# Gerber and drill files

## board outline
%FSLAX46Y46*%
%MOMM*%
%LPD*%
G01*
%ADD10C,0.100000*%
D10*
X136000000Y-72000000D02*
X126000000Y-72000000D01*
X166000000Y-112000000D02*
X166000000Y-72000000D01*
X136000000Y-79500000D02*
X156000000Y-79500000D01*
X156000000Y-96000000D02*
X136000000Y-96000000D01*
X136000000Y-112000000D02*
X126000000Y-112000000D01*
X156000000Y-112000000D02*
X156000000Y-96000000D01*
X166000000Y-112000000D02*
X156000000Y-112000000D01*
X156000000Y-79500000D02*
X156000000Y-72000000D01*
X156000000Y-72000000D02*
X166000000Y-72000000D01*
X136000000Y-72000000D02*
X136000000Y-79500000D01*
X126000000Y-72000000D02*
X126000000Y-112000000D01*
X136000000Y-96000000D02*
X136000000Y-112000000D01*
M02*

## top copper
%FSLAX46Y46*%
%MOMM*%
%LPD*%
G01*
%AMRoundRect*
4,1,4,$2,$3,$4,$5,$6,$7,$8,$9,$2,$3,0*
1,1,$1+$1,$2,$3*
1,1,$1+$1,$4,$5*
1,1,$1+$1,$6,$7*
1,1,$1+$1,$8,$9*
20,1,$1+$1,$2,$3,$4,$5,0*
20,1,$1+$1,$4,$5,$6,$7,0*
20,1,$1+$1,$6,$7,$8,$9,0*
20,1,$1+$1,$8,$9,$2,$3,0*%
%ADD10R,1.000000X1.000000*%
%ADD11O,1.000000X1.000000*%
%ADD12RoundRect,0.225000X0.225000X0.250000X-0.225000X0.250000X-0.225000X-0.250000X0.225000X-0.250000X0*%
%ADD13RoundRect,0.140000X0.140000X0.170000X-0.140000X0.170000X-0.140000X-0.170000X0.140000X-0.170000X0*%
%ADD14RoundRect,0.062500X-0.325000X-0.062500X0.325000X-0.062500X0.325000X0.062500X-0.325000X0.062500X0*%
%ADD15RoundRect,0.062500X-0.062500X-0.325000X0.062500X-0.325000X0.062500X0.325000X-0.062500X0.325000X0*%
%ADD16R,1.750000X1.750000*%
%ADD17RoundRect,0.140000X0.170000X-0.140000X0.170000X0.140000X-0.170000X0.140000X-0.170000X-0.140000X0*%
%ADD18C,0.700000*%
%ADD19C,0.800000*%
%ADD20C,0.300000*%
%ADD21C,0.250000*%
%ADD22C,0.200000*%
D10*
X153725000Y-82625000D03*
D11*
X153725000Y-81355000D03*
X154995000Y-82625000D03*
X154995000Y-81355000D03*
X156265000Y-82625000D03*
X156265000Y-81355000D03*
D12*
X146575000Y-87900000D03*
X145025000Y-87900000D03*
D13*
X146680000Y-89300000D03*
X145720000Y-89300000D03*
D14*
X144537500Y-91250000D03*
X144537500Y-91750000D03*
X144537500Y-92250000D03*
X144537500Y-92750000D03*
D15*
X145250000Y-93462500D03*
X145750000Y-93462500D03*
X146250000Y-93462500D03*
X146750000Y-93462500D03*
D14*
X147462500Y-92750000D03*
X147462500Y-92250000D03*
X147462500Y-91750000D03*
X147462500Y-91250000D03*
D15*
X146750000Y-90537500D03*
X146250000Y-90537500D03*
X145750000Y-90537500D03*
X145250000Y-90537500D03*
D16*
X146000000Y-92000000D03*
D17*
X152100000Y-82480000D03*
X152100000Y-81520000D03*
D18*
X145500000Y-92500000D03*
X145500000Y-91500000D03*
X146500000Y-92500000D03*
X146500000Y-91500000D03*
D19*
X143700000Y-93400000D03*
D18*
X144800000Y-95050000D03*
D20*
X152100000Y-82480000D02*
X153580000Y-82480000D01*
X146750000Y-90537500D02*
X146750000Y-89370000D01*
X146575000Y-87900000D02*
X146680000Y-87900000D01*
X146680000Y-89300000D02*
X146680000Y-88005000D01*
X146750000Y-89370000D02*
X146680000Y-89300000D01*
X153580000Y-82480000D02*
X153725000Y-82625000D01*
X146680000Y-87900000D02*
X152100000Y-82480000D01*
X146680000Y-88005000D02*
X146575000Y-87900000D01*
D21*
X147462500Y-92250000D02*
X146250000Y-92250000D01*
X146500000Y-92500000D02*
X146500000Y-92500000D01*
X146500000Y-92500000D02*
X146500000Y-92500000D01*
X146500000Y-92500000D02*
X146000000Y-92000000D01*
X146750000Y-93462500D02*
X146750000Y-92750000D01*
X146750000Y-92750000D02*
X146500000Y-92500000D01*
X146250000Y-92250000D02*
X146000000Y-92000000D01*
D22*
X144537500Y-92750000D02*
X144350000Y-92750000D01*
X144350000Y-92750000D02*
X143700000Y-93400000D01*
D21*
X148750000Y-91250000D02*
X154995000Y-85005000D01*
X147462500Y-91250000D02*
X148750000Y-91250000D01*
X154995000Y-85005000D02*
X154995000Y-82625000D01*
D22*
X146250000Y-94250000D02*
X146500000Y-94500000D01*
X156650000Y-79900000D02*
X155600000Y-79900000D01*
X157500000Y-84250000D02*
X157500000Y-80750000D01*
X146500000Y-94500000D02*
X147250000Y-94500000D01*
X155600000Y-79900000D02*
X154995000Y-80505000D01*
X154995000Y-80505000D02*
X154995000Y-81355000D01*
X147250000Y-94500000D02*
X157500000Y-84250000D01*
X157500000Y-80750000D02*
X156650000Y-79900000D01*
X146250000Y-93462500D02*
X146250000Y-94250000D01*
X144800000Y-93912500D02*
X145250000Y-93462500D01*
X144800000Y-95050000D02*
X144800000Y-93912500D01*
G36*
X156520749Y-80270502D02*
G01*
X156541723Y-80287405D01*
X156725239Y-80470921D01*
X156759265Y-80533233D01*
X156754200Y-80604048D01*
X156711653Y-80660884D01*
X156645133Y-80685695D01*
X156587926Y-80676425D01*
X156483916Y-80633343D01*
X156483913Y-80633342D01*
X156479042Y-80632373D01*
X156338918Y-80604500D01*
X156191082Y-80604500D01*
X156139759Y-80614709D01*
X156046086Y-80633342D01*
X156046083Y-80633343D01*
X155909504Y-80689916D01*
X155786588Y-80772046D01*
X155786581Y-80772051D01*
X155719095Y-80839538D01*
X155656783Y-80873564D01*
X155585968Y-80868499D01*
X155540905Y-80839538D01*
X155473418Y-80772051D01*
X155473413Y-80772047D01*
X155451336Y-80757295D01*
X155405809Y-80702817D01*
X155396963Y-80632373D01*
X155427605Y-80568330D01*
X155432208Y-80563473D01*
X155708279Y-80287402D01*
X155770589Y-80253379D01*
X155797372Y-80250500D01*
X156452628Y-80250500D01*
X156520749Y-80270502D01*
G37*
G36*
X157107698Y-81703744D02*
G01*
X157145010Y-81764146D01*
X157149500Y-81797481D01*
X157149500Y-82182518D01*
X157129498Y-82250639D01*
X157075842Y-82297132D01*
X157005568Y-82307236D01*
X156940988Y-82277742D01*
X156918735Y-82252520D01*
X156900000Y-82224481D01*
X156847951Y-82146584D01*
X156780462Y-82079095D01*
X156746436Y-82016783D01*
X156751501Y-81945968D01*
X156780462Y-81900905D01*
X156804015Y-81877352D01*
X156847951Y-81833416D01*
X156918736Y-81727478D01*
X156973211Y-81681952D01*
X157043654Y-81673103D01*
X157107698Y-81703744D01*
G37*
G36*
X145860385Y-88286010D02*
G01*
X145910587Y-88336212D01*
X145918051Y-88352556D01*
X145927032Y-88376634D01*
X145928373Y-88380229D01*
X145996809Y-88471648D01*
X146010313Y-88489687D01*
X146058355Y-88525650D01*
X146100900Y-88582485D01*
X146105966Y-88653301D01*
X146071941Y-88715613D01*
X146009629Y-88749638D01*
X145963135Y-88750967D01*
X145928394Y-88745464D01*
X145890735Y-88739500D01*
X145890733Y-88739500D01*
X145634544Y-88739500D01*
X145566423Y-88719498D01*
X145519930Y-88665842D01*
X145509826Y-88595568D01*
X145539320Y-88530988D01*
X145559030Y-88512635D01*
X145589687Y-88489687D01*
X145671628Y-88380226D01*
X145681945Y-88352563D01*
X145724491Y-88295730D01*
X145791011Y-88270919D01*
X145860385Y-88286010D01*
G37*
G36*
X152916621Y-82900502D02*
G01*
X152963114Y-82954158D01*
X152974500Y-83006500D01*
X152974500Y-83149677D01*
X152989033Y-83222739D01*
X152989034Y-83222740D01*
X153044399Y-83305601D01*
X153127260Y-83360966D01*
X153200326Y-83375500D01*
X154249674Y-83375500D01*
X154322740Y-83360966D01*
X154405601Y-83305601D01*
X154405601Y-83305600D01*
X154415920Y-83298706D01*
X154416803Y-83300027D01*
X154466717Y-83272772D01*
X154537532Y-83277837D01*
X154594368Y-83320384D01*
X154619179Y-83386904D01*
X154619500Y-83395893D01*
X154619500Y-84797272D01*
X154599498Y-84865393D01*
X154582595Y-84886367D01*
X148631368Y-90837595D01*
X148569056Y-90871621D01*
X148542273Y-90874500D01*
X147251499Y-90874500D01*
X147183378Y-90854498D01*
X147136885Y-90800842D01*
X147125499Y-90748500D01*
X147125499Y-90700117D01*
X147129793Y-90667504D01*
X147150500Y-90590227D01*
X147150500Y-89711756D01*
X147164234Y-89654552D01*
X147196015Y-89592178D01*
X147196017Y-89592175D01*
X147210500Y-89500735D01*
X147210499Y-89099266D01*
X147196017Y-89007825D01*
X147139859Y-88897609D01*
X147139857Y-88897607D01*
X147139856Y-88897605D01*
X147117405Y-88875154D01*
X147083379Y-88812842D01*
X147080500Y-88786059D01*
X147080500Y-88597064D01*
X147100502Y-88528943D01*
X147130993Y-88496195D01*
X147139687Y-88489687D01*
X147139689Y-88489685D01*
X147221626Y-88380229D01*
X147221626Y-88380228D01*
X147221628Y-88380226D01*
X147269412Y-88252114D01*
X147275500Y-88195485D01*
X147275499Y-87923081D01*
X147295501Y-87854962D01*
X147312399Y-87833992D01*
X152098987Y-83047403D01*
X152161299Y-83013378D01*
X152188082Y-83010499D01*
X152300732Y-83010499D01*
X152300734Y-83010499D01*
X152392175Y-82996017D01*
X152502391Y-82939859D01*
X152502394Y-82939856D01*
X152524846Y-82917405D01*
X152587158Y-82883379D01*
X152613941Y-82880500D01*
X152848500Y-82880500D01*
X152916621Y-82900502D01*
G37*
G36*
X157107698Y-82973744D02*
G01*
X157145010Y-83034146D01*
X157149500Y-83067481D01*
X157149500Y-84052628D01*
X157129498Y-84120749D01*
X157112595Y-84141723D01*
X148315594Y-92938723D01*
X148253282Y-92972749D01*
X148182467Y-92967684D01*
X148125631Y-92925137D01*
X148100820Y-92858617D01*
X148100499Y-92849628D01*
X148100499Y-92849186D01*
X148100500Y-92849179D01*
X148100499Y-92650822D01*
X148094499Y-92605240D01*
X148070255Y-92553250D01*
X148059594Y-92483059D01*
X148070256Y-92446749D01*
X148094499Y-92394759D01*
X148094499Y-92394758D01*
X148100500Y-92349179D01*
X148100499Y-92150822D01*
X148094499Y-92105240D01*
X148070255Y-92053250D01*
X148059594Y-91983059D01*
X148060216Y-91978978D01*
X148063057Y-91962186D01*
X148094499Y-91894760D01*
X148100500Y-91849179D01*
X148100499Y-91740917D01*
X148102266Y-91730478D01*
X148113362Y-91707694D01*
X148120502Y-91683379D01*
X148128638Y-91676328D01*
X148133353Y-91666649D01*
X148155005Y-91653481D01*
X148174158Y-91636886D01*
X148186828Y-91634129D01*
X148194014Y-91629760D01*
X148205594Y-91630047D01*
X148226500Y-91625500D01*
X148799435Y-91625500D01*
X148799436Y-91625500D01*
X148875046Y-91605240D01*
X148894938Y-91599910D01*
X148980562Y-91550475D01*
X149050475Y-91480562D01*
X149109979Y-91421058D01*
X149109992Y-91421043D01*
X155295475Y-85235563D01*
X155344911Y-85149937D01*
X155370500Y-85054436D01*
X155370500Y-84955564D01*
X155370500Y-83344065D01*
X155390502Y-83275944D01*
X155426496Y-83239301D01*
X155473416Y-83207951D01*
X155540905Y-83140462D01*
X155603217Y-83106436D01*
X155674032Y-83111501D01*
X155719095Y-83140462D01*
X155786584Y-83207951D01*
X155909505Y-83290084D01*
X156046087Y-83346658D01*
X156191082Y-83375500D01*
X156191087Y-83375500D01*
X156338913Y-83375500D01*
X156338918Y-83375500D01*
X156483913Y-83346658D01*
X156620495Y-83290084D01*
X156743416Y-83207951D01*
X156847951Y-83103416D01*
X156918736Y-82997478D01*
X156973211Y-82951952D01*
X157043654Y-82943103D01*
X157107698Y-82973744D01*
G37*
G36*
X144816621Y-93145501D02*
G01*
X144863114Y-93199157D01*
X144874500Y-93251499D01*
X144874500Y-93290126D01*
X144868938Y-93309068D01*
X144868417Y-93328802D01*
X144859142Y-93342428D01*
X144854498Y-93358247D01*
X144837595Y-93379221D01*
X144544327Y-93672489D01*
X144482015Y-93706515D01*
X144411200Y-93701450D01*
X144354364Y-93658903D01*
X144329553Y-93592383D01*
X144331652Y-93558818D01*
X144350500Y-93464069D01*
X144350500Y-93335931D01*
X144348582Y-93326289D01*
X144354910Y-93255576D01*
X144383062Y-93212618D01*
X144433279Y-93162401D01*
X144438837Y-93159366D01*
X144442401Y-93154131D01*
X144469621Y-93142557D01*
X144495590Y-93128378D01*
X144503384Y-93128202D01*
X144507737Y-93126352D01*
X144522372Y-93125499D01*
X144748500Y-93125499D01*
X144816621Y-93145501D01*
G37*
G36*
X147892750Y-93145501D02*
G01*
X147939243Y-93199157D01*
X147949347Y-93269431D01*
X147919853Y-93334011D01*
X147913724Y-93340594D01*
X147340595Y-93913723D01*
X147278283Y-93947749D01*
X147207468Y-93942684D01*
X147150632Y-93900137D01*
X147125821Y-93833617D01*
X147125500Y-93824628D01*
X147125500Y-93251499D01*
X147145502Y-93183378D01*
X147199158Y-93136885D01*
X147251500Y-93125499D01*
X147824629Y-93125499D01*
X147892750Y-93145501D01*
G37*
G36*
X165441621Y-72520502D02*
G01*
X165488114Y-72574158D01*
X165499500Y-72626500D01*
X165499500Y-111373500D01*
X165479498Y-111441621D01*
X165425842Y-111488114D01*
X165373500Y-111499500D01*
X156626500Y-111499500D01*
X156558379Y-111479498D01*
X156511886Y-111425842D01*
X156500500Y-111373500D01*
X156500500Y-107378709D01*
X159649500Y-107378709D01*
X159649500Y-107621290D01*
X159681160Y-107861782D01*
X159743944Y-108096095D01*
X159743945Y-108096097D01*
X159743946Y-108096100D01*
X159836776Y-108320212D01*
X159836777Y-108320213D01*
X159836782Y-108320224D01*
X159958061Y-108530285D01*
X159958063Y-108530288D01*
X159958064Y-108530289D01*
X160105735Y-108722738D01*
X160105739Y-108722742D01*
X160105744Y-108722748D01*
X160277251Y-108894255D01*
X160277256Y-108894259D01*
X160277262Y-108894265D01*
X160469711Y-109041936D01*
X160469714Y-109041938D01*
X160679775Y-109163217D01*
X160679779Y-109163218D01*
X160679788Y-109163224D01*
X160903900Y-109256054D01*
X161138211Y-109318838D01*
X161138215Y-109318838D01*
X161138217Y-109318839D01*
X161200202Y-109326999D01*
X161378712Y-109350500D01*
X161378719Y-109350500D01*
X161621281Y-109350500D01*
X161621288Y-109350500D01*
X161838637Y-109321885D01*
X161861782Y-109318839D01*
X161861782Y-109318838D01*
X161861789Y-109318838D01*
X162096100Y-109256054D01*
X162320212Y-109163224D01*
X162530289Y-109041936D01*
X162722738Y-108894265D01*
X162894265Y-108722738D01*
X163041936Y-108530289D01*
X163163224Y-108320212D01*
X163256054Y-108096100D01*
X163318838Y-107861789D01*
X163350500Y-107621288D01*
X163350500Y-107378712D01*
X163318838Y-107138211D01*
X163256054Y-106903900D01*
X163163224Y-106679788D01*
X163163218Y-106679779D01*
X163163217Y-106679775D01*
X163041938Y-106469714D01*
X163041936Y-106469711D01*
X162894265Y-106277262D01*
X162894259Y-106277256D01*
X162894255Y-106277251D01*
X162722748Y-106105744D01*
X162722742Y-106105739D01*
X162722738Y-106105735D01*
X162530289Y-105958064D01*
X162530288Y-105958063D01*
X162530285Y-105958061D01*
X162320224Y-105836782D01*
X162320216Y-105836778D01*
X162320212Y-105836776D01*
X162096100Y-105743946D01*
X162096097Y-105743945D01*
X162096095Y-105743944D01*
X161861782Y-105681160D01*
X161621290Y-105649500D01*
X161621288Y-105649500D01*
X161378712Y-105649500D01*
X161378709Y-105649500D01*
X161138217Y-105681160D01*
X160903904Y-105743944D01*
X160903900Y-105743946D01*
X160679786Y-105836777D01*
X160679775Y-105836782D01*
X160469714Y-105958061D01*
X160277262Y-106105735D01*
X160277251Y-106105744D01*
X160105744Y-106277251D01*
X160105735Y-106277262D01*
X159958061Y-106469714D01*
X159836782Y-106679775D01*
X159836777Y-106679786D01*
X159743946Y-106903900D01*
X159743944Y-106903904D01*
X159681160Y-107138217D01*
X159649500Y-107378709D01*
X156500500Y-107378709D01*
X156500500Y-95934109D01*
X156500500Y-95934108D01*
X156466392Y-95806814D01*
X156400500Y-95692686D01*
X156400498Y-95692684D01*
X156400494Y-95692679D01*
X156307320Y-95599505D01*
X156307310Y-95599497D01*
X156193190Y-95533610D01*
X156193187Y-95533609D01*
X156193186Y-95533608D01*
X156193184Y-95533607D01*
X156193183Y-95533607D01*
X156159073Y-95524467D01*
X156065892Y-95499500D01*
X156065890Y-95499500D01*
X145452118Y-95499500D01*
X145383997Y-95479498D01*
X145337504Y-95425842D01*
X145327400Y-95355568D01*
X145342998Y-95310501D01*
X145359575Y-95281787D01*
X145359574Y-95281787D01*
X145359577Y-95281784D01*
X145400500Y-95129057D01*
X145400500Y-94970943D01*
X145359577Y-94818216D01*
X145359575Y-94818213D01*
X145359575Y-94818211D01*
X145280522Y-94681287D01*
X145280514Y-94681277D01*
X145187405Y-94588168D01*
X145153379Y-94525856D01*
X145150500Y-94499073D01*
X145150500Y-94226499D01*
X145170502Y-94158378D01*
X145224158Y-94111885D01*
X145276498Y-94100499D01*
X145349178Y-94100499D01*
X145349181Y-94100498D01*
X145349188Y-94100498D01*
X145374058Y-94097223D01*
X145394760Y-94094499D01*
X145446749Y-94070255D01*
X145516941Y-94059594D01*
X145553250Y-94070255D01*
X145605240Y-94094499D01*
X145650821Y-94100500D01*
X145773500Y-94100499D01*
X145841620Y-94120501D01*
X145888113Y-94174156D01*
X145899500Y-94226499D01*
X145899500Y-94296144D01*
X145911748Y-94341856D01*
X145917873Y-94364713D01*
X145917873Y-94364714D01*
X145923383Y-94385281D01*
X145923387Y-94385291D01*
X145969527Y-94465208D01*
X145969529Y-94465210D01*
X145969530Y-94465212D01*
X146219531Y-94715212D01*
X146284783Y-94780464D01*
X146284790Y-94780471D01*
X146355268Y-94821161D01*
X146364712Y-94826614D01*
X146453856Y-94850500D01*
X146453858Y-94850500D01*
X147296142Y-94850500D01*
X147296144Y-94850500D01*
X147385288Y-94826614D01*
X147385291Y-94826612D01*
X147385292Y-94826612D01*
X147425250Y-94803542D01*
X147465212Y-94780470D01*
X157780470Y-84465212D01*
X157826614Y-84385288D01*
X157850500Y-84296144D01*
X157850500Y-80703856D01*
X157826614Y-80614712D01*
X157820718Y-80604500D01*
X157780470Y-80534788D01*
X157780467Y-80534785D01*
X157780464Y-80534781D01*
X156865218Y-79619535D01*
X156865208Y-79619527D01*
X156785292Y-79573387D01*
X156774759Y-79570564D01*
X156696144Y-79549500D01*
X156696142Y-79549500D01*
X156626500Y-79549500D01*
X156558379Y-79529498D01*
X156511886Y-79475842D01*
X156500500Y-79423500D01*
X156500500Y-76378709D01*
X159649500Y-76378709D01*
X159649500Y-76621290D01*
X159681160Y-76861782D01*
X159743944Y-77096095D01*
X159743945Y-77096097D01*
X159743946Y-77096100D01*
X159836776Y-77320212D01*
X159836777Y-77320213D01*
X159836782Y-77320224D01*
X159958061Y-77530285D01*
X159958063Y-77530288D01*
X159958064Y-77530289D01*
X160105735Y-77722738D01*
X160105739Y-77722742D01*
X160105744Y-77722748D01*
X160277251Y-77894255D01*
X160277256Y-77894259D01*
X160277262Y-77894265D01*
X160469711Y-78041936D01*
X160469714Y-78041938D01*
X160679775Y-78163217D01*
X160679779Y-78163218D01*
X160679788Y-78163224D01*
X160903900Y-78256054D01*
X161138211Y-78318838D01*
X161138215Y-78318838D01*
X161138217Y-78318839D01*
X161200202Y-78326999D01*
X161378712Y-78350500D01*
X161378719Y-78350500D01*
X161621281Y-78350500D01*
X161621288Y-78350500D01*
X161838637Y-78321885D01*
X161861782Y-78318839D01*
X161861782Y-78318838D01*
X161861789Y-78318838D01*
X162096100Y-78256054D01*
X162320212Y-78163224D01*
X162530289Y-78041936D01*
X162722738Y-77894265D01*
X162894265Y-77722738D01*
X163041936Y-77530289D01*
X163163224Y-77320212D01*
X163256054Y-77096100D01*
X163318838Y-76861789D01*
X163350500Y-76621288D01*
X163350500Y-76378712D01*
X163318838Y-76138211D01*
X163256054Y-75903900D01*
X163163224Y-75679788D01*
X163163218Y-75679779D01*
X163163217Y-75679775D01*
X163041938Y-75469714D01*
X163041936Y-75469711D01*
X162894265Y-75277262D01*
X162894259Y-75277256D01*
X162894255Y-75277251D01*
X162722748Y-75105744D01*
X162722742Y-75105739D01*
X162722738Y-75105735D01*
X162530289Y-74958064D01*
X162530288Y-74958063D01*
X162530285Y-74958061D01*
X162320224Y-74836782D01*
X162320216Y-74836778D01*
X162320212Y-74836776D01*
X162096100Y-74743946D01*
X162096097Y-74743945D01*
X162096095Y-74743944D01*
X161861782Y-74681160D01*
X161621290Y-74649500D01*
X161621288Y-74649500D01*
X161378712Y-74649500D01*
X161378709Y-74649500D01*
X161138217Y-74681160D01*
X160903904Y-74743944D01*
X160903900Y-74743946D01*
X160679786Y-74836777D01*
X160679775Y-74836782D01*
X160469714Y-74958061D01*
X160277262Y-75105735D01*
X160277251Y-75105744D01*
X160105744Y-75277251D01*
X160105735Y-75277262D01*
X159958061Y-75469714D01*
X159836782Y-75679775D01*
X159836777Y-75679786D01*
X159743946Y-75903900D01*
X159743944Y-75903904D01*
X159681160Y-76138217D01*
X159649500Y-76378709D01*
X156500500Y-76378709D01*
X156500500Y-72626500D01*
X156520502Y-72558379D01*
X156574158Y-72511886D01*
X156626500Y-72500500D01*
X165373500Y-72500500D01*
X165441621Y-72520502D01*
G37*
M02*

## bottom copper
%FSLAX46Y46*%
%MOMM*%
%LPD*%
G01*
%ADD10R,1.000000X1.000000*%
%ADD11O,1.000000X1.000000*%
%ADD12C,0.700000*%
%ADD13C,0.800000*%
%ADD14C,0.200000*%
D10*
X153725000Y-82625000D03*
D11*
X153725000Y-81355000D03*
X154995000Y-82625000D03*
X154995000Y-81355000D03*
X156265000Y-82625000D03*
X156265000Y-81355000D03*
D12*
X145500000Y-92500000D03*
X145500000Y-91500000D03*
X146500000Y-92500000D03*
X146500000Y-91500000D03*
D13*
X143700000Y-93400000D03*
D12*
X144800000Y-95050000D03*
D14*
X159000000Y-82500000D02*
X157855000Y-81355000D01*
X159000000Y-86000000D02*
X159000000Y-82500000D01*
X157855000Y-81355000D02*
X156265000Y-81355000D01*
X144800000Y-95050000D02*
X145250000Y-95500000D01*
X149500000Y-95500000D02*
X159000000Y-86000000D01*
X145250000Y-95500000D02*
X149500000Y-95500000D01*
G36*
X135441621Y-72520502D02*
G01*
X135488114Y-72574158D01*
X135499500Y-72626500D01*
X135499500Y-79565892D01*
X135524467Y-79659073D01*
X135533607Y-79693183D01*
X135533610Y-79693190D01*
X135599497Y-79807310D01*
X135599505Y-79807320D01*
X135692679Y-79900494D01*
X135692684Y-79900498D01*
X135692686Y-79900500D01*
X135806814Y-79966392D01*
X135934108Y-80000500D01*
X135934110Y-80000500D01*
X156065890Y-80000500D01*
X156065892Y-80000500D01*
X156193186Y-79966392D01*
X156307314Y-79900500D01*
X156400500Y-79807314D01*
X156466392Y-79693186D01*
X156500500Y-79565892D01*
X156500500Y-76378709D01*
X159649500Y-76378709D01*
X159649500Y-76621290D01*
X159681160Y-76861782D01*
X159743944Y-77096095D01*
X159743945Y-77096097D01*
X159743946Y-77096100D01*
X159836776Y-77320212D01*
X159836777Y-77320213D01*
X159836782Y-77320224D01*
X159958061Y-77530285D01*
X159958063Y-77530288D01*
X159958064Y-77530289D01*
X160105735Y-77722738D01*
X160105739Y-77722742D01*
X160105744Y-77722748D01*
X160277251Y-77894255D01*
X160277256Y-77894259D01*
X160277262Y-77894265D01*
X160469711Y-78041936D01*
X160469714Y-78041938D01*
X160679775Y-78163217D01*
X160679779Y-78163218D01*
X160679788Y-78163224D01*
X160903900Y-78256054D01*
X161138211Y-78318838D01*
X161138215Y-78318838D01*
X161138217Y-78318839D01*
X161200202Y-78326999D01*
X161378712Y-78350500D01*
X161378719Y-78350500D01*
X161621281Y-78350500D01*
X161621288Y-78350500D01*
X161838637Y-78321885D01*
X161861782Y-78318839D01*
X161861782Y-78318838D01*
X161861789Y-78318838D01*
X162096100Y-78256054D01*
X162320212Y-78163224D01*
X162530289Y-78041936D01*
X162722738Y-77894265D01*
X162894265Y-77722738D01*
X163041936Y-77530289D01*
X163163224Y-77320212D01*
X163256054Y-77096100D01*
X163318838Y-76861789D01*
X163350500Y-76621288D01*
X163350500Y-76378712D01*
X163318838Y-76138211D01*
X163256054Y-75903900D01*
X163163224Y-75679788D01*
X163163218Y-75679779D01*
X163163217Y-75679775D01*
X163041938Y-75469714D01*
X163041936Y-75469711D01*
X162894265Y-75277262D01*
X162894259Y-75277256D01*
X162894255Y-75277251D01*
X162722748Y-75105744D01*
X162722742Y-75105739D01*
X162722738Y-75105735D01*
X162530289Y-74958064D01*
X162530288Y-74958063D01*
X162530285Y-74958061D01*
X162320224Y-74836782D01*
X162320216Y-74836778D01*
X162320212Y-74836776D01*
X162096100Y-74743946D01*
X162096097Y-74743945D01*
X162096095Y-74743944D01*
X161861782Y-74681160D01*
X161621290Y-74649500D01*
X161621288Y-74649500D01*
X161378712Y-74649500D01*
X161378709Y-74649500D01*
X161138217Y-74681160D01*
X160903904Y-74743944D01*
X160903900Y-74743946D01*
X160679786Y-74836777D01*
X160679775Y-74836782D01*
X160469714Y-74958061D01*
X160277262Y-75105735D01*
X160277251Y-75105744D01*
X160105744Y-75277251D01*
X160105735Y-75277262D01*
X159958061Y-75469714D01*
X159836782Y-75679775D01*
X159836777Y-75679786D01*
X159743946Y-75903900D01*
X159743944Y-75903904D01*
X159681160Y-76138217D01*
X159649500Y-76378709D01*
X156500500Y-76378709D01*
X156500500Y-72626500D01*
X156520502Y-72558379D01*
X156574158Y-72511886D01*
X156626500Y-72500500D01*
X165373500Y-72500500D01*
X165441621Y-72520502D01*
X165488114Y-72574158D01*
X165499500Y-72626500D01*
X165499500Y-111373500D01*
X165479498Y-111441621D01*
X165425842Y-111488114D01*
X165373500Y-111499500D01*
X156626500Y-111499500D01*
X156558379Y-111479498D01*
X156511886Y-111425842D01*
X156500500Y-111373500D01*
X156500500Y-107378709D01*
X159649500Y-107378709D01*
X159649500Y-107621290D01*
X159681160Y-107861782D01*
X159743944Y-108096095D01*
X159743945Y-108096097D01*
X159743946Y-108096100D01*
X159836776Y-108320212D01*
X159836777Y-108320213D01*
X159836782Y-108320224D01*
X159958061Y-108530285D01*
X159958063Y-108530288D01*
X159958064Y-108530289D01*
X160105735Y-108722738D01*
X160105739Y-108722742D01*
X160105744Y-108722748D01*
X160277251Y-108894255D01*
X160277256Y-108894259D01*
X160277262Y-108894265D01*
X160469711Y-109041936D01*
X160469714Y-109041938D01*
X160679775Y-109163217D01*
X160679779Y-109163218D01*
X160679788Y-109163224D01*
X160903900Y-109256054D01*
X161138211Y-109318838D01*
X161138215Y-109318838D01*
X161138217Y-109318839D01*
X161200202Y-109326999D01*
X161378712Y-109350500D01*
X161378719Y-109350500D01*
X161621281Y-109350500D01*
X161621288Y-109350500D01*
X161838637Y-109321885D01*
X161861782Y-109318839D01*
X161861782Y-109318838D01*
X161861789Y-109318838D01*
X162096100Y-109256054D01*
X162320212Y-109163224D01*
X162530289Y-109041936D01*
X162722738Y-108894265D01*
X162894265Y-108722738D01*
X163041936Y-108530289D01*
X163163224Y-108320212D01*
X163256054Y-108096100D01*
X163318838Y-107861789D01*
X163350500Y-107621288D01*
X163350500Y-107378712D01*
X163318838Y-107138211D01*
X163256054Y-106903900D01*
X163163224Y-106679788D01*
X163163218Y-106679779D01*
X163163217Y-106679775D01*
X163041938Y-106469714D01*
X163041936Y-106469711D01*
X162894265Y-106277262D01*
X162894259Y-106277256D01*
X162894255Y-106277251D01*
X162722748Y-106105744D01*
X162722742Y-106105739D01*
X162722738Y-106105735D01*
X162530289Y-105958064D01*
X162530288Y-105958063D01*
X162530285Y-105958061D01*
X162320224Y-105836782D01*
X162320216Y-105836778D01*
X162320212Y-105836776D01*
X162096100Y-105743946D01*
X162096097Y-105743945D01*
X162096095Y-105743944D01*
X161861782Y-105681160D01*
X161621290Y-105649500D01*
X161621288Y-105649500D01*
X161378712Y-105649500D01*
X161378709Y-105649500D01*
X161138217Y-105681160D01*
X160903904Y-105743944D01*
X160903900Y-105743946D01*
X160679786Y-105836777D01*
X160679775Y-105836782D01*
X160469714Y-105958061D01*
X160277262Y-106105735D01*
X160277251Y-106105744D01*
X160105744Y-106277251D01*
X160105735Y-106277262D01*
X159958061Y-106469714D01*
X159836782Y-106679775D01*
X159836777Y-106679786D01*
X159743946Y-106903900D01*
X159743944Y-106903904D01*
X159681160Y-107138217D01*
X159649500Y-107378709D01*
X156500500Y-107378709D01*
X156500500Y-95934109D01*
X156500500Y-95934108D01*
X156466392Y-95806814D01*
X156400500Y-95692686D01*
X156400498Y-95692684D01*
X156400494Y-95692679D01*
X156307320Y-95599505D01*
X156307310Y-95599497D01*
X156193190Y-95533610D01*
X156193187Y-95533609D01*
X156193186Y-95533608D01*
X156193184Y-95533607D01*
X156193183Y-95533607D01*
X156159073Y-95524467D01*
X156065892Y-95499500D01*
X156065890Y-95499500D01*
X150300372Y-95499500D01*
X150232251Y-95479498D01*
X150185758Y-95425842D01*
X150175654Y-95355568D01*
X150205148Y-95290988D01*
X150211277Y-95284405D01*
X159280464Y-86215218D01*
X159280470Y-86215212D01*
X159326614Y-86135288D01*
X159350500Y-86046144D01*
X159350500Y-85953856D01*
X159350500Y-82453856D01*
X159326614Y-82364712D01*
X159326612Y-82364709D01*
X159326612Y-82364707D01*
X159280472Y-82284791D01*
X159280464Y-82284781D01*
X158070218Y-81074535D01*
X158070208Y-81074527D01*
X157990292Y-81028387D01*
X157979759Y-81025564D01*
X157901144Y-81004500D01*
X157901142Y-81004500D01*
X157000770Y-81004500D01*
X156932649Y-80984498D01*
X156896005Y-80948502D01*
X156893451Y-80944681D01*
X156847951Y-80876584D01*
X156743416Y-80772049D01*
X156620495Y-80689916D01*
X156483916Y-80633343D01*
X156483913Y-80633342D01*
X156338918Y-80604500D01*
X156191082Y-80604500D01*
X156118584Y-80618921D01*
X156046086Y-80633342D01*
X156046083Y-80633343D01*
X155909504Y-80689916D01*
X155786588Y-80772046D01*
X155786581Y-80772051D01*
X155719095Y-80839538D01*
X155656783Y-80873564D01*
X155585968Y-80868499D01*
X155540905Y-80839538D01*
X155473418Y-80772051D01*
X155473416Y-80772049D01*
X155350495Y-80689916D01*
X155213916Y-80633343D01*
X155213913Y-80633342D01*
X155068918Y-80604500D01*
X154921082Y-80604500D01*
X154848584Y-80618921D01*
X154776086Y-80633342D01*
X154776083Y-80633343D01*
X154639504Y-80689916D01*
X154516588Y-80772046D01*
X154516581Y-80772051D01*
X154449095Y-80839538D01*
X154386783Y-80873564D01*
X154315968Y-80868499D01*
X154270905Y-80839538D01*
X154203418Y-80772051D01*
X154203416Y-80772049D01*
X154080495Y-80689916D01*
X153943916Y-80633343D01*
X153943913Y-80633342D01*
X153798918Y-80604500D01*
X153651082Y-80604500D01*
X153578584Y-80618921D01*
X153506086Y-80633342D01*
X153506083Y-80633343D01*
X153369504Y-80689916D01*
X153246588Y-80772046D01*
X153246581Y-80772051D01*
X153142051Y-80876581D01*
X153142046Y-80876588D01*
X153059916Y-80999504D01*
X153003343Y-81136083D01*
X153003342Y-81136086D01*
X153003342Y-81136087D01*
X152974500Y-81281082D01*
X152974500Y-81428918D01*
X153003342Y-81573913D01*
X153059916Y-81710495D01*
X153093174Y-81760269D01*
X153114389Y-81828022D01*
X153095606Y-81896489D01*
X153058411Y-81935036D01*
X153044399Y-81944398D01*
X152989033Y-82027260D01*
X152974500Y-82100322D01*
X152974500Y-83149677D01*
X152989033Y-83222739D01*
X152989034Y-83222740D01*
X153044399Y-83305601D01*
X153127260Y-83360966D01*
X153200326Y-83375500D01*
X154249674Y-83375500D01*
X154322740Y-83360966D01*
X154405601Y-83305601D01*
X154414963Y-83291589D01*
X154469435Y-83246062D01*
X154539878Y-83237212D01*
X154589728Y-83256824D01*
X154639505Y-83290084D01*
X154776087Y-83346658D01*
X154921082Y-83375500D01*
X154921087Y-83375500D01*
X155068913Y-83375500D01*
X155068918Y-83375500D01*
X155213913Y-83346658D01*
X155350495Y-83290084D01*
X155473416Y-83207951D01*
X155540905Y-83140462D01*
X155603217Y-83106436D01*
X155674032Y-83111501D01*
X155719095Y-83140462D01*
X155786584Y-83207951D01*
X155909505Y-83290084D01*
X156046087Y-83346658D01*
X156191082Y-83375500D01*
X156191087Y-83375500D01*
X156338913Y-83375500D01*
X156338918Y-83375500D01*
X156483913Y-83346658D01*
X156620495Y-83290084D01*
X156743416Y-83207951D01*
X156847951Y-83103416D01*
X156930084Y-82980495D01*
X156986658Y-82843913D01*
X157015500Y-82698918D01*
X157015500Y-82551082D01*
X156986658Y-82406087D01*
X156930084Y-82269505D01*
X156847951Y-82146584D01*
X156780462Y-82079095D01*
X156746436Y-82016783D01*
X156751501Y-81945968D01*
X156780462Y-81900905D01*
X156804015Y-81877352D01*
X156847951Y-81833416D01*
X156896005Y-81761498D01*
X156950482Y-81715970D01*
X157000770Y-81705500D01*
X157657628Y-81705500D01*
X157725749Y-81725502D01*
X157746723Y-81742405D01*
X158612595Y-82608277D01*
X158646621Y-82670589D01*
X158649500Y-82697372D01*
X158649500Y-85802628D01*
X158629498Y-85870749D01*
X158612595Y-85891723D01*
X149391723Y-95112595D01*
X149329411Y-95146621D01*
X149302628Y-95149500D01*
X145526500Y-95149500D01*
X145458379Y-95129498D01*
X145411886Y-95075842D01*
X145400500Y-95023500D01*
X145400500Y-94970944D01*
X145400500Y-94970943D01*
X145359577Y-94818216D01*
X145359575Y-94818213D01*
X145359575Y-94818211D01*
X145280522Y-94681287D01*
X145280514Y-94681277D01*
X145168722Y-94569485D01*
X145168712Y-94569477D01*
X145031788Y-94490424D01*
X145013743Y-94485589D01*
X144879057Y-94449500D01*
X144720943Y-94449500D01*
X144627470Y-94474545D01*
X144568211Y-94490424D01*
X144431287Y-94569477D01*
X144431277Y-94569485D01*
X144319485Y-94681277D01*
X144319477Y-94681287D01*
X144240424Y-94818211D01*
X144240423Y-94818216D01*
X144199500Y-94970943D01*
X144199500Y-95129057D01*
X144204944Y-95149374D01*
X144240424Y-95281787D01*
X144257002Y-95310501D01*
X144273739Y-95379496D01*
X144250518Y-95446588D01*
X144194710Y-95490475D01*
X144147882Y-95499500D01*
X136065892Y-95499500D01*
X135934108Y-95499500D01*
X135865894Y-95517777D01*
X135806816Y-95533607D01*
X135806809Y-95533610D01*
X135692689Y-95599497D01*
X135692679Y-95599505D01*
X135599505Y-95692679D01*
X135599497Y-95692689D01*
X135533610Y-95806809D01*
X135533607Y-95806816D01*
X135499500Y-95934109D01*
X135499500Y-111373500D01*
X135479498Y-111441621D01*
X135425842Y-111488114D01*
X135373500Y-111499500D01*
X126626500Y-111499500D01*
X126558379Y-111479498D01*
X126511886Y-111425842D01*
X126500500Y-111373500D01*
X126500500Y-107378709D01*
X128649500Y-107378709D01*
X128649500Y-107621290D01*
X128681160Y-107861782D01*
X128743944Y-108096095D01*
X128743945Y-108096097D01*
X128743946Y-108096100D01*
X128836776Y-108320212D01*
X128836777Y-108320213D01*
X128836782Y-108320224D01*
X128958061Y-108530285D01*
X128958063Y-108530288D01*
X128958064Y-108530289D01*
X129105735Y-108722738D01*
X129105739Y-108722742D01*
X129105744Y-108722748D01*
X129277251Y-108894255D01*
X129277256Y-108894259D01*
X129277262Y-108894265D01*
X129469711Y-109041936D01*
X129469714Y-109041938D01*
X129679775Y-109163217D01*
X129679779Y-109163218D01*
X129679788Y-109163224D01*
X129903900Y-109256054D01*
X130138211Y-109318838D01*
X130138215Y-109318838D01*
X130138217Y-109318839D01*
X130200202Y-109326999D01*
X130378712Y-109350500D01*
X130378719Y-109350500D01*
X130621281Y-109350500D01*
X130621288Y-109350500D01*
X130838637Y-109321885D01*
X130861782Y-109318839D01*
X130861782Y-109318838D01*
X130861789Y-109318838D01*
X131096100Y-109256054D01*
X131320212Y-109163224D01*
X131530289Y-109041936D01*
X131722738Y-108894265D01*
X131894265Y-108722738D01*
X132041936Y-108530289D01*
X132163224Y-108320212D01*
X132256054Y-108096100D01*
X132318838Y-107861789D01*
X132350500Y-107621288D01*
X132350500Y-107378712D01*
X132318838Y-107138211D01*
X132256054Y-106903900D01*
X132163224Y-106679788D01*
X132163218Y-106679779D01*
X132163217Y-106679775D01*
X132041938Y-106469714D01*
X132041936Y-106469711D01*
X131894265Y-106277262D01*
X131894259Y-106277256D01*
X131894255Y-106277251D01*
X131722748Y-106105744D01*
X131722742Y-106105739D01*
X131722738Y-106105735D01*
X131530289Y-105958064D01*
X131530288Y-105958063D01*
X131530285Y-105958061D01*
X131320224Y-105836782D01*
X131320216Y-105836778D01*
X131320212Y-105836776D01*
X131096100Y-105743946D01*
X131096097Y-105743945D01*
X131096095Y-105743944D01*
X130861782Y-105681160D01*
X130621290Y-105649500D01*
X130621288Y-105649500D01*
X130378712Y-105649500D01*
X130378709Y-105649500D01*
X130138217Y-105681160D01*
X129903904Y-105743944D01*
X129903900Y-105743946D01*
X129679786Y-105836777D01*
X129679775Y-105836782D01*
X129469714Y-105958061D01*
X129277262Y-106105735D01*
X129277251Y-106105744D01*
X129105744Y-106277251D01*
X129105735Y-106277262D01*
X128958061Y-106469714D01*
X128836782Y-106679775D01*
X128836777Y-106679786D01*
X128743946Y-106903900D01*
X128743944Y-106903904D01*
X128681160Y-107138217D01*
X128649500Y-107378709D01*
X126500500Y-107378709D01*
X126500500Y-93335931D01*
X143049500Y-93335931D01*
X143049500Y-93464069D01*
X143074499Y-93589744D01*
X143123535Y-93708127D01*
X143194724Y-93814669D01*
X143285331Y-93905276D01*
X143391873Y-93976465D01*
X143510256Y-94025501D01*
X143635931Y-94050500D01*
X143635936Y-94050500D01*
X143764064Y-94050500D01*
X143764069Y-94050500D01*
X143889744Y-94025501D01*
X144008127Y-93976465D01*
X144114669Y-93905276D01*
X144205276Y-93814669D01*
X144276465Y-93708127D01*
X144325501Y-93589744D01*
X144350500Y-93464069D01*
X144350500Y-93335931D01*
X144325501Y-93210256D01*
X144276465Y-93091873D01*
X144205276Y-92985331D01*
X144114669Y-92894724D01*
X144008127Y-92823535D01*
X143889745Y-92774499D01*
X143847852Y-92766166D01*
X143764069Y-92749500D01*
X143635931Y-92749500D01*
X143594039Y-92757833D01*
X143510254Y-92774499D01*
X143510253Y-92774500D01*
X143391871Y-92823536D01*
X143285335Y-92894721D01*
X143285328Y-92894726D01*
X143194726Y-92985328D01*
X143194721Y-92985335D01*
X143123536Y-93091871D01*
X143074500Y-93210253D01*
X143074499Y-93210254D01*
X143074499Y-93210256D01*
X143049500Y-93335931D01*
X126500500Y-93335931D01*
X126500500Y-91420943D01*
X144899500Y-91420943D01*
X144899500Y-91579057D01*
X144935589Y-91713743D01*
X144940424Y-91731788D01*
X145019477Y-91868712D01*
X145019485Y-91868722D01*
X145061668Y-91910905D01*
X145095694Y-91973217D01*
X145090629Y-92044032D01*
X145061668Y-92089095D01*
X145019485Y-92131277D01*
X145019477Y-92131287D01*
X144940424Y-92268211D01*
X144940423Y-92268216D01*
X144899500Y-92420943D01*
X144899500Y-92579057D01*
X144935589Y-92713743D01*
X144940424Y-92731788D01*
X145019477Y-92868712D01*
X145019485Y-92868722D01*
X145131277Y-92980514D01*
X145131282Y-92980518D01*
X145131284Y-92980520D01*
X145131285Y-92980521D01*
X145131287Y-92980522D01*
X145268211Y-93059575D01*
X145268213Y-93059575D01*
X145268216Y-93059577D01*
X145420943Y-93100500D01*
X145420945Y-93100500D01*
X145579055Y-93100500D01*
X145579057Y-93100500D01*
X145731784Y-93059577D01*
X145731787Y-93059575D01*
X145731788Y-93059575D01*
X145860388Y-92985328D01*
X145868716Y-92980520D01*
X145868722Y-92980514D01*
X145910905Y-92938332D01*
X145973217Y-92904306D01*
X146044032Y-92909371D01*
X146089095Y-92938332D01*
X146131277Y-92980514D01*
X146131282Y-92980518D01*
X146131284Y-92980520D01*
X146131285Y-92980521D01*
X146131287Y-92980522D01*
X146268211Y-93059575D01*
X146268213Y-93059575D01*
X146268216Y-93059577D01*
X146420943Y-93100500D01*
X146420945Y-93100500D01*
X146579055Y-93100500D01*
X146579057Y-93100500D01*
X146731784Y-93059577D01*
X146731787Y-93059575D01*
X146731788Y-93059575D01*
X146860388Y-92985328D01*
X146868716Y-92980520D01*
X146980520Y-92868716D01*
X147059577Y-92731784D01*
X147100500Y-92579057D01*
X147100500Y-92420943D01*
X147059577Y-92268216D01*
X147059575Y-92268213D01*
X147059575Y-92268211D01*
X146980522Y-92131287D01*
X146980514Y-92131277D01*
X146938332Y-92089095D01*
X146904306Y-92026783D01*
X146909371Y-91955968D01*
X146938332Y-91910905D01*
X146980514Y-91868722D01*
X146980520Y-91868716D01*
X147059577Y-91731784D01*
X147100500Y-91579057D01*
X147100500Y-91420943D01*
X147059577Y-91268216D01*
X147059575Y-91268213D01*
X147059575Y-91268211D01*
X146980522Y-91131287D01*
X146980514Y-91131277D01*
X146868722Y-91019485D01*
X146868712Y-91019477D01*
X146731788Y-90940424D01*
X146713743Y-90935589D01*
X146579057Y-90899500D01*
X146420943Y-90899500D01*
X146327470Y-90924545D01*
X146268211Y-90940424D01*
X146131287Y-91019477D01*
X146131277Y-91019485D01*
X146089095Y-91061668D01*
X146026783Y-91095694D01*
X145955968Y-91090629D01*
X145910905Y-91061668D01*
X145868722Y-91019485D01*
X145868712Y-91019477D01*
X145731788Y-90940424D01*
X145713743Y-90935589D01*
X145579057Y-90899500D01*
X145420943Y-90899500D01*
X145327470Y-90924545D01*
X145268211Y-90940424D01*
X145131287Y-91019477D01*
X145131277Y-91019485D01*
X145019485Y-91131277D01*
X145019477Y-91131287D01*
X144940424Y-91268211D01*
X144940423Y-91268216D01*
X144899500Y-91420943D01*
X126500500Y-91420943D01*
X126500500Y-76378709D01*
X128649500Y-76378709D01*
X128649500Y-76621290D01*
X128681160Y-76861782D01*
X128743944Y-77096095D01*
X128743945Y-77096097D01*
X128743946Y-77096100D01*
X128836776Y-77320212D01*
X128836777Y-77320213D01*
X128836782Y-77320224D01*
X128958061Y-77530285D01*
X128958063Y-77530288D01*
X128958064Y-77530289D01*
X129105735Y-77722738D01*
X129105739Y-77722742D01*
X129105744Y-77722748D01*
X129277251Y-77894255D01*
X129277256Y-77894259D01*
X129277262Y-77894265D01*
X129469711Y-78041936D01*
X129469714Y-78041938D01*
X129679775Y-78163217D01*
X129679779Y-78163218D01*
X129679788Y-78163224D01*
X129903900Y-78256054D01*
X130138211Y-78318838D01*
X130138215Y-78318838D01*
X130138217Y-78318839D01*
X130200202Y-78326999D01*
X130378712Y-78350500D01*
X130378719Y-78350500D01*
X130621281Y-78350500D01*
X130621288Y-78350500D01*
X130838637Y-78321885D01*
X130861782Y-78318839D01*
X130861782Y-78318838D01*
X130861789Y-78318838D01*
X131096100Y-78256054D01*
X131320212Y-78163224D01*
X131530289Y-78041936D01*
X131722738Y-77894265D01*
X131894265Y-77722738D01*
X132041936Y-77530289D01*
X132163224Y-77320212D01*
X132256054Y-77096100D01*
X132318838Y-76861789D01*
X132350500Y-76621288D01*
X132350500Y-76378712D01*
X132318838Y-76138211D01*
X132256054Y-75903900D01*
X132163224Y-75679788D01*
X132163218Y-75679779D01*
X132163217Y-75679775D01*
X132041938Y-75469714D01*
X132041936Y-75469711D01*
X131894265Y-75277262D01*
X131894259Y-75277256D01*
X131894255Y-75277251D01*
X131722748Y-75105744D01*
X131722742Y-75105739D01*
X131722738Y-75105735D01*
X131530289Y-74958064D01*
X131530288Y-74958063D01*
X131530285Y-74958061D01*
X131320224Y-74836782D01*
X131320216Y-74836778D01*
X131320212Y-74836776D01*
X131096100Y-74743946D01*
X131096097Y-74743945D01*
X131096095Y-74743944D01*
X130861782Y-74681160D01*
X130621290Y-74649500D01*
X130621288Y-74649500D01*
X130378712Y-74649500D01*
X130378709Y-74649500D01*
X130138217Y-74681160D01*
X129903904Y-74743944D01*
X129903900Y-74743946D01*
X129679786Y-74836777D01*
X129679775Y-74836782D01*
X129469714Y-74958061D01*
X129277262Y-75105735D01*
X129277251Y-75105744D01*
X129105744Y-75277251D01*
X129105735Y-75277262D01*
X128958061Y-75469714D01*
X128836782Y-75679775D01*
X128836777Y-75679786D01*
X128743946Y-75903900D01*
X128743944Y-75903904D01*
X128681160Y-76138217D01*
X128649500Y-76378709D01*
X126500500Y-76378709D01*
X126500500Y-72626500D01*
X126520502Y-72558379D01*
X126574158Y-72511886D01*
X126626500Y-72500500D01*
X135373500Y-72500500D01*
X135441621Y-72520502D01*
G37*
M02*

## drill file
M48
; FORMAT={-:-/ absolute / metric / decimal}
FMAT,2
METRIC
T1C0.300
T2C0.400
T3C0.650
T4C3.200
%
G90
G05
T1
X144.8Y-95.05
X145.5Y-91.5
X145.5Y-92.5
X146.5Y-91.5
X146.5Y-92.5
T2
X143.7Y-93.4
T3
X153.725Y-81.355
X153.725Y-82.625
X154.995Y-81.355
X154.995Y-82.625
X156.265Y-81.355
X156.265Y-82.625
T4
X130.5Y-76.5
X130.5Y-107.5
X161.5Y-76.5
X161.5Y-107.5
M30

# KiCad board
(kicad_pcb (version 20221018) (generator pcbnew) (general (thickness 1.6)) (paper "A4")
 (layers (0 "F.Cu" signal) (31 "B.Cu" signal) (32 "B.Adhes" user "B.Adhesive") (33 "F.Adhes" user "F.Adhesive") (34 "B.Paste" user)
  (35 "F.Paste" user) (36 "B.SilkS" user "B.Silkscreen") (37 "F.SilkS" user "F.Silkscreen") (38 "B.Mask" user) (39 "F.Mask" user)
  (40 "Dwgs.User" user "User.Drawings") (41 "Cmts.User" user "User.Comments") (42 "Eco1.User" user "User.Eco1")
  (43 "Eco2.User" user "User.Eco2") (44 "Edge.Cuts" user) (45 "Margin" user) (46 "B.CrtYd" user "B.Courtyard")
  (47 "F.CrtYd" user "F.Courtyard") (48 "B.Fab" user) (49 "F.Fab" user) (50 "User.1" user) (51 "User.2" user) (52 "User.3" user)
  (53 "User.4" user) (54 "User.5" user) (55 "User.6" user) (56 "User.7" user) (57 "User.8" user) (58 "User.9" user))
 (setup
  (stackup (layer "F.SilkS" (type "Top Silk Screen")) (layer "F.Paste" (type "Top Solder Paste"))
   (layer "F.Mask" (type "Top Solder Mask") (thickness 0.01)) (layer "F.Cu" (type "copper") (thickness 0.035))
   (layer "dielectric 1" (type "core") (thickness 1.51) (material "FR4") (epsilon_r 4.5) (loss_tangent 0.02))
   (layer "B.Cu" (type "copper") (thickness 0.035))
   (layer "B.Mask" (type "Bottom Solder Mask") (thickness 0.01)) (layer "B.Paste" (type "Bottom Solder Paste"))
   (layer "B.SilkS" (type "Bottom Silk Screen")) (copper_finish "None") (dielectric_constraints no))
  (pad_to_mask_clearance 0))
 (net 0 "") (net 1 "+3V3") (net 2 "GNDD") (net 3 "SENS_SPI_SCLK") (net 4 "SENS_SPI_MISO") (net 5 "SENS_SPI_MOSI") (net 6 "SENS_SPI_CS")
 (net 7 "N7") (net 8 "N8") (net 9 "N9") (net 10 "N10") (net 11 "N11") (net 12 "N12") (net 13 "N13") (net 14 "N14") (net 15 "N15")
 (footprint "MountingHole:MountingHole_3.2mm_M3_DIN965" (layer "F.Cu") (at 130.5 76.5)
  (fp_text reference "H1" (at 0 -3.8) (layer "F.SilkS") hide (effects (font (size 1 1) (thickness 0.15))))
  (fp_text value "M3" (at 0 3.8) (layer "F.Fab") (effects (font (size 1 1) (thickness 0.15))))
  (pad "" np_thru_hole circle (at 0 0) (size 3.2 3.2) (drill 3.2) (layers "*.Cu" "*.Mask")))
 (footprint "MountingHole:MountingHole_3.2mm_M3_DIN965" (layer "F.Cu") (at 161.5 76.5)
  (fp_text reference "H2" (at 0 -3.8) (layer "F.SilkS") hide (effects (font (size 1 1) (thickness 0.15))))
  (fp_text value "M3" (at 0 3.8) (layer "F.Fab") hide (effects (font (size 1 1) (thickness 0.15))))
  (pad "" np_thru_hole circle (at 0 0) (size 3.2 3.2) (drill 3.2) (layers "*.Cu" "*.Mask")))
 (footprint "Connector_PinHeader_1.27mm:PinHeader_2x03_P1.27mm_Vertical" (layer "F.Cu") (at 153.725 82.625 90)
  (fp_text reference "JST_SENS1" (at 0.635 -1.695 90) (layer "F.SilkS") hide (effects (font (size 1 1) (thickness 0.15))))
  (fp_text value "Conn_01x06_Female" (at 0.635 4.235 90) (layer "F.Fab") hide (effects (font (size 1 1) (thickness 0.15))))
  (pad "1" thru_hole rect (at 0 0 90) (size 1 1) (drill 0.65) (layers "*.Cu" "*.Mask") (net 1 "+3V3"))
  (pad "2" thru_hole oval (at 1.27 0 90) (size 1 1) (drill 0.65) (layers "*.Cu" "*.Mask") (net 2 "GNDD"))
  (pad "3" thru_hole oval (at 0 1.27 90) (size 1 1) (drill 0.65) (layers "*.Cu" "*.Mask") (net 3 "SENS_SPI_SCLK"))
  (pad "4" thru_hole oval (at 1.27 1.27 90) (size 1 1) (drill 0.65) (layers "*.Cu" "*.Mask") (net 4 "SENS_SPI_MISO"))
  (pad "5" thru_hole oval (at 0 2.54 90) (size 1 1) (drill 0.65) (layers "*.Cu" "*.Mask") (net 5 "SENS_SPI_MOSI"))
  (pad "6" thru_hole oval (at 1.27 2.54 90) (size 1 1) (drill 0.65) (layers "*.Cu" "*.Mask") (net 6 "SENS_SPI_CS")))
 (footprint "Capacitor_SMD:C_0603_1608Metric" (layer "F.Cu") (at 145.8 87.9 180)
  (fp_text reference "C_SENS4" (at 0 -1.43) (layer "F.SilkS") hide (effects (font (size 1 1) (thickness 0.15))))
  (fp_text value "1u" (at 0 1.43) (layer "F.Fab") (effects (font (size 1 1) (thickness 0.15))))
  (pad "1" smd roundrect (at -0.775 0 180) (size 0.9 0.95) (layers "F.Cu" "F.Paste" "F.Mask") (roundrect_rratio 0.25) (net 1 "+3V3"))
  (pad "2" smd roundrect (at 0.775 0 180) (size 0.9 0.95) (layers "F.Cu" "F.Paste" "F.Mask") (roundrect_rratio 0.25) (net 2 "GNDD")))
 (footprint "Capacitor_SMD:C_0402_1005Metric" (layer "F.Cu") (at 146.2 89.3 180)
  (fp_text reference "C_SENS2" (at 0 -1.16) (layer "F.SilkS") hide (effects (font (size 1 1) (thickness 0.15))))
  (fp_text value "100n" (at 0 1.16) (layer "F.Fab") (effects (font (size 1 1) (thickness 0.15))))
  (pad "1" smd roundrect (at -0.48 0 180) (size 0.56 0.62) (layers "F.Cu" "F.Paste" "F.Mask") (roundrect_rratio 0.25) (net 1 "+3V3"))
  (pad "2" smd roundrect (at 0.48 0 180) (size 0.56 0.62) (layers "F.Cu" "F.Paste" "F.Mask") (roundrect_rratio 0.25) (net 2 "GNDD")))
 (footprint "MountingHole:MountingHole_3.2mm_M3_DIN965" (layer "F.Cu") (at 161.5 107.5)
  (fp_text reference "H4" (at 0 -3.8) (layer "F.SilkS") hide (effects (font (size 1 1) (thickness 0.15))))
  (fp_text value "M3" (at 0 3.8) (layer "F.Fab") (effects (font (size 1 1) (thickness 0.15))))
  (pad "" np_thru_hole circle (at 0 0) (size 3.2 3.2) (drill 3.2) (layers "*.Cu" "*.Mask")))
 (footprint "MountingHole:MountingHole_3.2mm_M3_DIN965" (layer "F.Cu") (at 130.5 107.5)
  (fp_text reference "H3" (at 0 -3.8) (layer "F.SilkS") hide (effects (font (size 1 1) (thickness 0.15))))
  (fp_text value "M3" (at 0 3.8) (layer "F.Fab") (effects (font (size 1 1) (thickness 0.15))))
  (pad "" np_thru_hole circle (at 0 0) (size 3.2 3.2) (drill 3.2) (layers "*.Cu" "*.Mask")))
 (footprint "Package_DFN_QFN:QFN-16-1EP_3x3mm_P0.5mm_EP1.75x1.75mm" (layer "F.Cu") (at 146 92)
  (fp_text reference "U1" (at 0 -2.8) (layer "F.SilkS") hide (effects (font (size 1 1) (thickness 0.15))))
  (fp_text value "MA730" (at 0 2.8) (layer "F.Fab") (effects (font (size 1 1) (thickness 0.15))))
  (pad "" smd roundrect (at -0.44 -0.44) (size 0.71 0.71) (layers "F.Paste") (roundrect_rratio 0.25))
  (pad "" smd roundrect (at -0.44 0.44) (size 0.71 0.71) (layers "F.Paste") (roundrect_rratio 0.25))
  (pad "" smd roundrect (at 0.44 -0.44) (size 0.71 0.71) (layers "F.Paste") (roundrect_rratio 0.25))
  (pad "" smd roundrect (at 0.44 0.44) (size 0.71 0.71) (layers "F.Paste") (roundrect_rratio 0.25))
  (pad "1" smd roundrect (at -1.4625 -0.75) (size 0.775 0.25) (layers "F.Cu" "F.Paste" "F.Mask") (roundrect_rratio 0.25) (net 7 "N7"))
  (pad "2" smd roundrect (at -1.4625 -0.25) (size 0.775 0.25) (layers "F.Cu" "F.Paste" "F.Mask") (roundrect_rratio 0.25) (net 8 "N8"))
  (pad "3" smd roundrect (at -1.4625 0.25) (size 0.775 0.25) (layers "F.Cu" "F.Paste" "F.Mask") (roundrect_rratio 0.25) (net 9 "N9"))
  (pad "4" smd roundrect (at -1.4625 0.75) (size 0.775 0.25) (layers "F.Cu" "F.Paste" "F.Mask") (roundrect_rratio 0.25)
   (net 5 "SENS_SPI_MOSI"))
  (pad "5" smd roundrect (at -0.75 1.4625) (size 0.25 0.775) (layers "F.Cu" "F.Paste" "F.Mask") (roundrect_rratio 0.25)
   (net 6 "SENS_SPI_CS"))
  (pad "6" smd roundrect (at -0.25 1.4625) (size 0.25 0.775) (layers "F.Cu" "F.Paste" "F.Mask") (roundrect_rratio 0.25) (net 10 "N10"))
  (pad "7" smd roundrect (at 0.25 1.4625) (size 0.25 0.775) (layers "F.Cu" "F.Paste" "F.Mask") (roundrect_rratio 0.25)
   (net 4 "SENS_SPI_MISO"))
  (pad "8" smd roundrect (at 0.75 1.4625) (size 0.25 0.775) (layers "F.Cu" "F.Paste" "F.Mask") (roundrect_rratio 0.25) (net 2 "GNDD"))
  (pad "9" smd roundrect (at 1.4625 0.75) (size 0.775 0.25) (layers "F.Cu" "F.Paste" "F.Mask") (roundrect_rratio 0.25) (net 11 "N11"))
  (pad "10" smd roundrect (at 1.4625 0.25) (size 0.775 0.25) (layers "F.Cu" "F.Paste" "F.Mask") (roundrect_rratio 0.25) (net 2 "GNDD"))
  (pad "11" smd roundrect (at 1.4625 -0.25) (size 0.775 0.25) (layers "F.Cu" "F.Paste" "F.Mask") (roundrect_rratio 0.25) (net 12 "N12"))
  (pad "12" smd roundrect (at 1.4625 -0.75) (size 0.775 0.25) (layers "F.Cu" "F.Paste" "F.Mask") (roundrect_rratio 0.25)
   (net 3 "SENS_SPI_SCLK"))
  (pad "13" smd roundrect (at 0.75 -1.4625) (size 0.25 0.775) (layers "F.Cu" "F.Paste" "F.Mask") (roundrect_rratio 0.25) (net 1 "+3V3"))
  (pad "14" smd roundrect (at 0.25 -1.4625) (size 0.25 0.775) (layers "F.Cu" "F.Paste" "F.Mask") (roundrect_rratio 0.25) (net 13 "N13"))
  (pad "15" smd roundrect (at -0.25 -1.4625) (size 0.25 0.775) (layers "F.Cu" "F.Paste" "F.Mask") (roundrect_rratio 0.25) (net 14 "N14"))
  (pad "16" smd roundrect (at -0.75 -1.4625) (size 0.25 0.775) (layers "F.Cu" "F.Paste" "F.Mask") (roundrect_rratio 0.25) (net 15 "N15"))
  (pad "17" smd rect (at 0 0) (size 1.75 1.75) (layers "F.Cu" "F.Mask") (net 2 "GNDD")))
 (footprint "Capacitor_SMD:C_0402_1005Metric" (layer "F.Cu") (at 152.1 82 90)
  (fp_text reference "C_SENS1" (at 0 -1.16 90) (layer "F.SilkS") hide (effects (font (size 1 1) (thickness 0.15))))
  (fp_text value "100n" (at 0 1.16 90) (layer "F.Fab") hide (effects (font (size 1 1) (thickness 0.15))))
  (pad "1" smd roundrect (at -0.48 0 90) (size 0.56 0.62) (layers "F.Cu" "F.Paste" "F.Mask") (roundrect_rratio 0.25) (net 1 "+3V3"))
  (pad "2" smd roundrect (at 0.48 0 90) (size 0.56 0.62) (layers "F.Cu" "F.Paste" "F.Mask") (roundrect_rratio 0.25) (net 2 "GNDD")))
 (gr_line (start 136 72) (end 126 72) (stroke (width 0.1) (type default)) (layer "Edge.Cuts"))
 (gr_line (start 166 112) (end 166 72) (stroke (width 0.1) (type solid)) (layer "Edge.Cuts"))
 (gr_line (start 136 79.5) (end 156 79.5) (stroke (width 0.1) (type default)) (layer "Edge.Cuts"))
 (gr_line (start 156 96) (end 136 96) (stroke (width 0.1) (type default)) (layer "Edge.Cuts"))
 (gr_line (start 136 112) (end 126 112) (stroke (width 0.1) (type default)) (layer "Edge.Cuts"))
 (gr_line (start 156 112) (end 156 96) (stroke (width 0.1) (type default)) (layer "Edge.Cuts"))
 (gr_line (start 166 112) (end 156 112) (stroke (width 0.1) (type default)) (layer "Edge.Cuts"))
 (gr_line (start 156 79.5) (end 156 72) (stroke (width 0.1) (type default)) (layer "Edge.Cuts"))
 (gr_line (start 156 72) (end 166 72) (stroke (width 0.1) (type default)) (layer "Edge.Cuts"))
 (gr_line (start 136 72) (end 136 79.5) (stroke (width 0.1) (type default)) (layer "Edge.Cuts"))
 (gr_line (start 126 72) (end 126 112) (stroke (width 0.1) (type solid)) (layer "Edge.Cuts"))
 (gr_line (start 136 96) (end 136 112) (stroke (width 0.1) (type default)) (layer "Edge.Cuts"))
 (segment (start 152.1 82.48) (end 153.58 82.48) (width 0.3) (layer "F.Cu") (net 1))
 (segment (start 146.75 90.5375) (end 146.75 89.37) (width 0.3) (layer "F.Cu") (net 1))
 (segment (start 146.575 87.9) (end 146.68 87.9) (width 0.3) (layer "F.Cu") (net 1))
 (segment (start 146.68 89.3) (end 146.68 88.005) (width 0.3) (layer "F.Cu") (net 1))
 (segment (start 146.75 89.37) (end 146.68 89.3) (width 0.3) (layer "F.Cu") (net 1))
 (segment (start 153.58 82.48) (end 153.725 82.625) (width 0.3) (layer "F.Cu") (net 1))
 (segment (start 146.68 87.9) (end 152.1 82.48) (width 0.3) (layer "F.Cu") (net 1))
 (segment (start 146.68 88.005) (end 146.575 87.9) (width 0.3) (layer "F.Cu") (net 1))
 (segment (start 147.4625 92.25) (end 146.25 92.25) (width 0.25) (layer "F.Cu") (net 2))
 (segment (start 146.5 92.5) (end 146.5 92.5) (width 0.25) (layer "F.Cu") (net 2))
 (segment (start 146.5 92.5) (end 146.5 92.5) (width 0.25) (layer "F.Cu") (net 2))
 (segment (start 146.5 92.5) (end 146 92) (width 0.25) (layer "F.Cu") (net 2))
 (segment (start 146.75 93.4625) (end 146.75 92.75) (width 0.25) (layer "F.Cu") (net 2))
 (segment (start 146.75 92.75) (end 146.5 92.5) (width 0.25) (layer "F.Cu") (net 2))
 (segment (start 146.25 92.25) (end 146 92) (width 0.25) (layer "F.Cu") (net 2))
 (via (at 145.5 92.5) (size 0.7) (drill 0.3) (layers "F.Cu" "B.Cu") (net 2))
 (via (at 145.5 91.5) (size 0.7) (drill 0.3) (layers "F.Cu" "B.Cu") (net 2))
 (via (at 146.5 92.5) (size 0.7) (drill 0.3) (layers "F.Cu" "B.Cu") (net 2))
 (via (at 146.5 91.5) (size 0.7) (drill 0.3) (layers "F.Cu" "B.Cu") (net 2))
 (segment (start 144.5375 92.75) (end 144.35 92.75) (width 0.2) (layer "F.Cu") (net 5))
 (segment (start 144.35 92.75) (end 143.7 93.4) (width 0.2) (layer "F.Cu") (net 5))
 (via (at 143.7 93.4) (size 0.8) (drill 0.4) (layers "F.Cu" "B.Cu") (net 5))
 (segment (start 148.75 91.25) (end 154.995 85.005) (width 0.25) (layer "F.Cu") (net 3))
 (segment (start 147.4625 91.25) (end 148.75 91.25) (width 0.25) (layer "F.Cu") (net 3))
 (segment (start 154.995 85.005) (end 154.995 82.625) (width 0.25) (layer "F.Cu") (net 3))
 (segment (start 146.25 94.25) (end 146.5 94.5) (width 0.2) (layer "F.Cu") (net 4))
 (segment (start 156.65 79.9) (end 155.6 79.9) (width 0.2) (layer "F.Cu") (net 4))
 (segment (start 157.5 84.25) (end 157.5 80.75) (width 0.2) (layer "F.Cu") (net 4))
 (segment (start 146.5 94.5) (end 147.25 94.5) (width 0.2) (layer "F.Cu") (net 4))
 (segment (start 155.6 79.9) (end 154.995 80.505) (width 0.2) (layer "F.Cu") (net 4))
 (segment (start 154.995 80.505) (end 154.995 81.355) (width 0.2) (layer "F.Cu") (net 4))
 (segment (start 147.25 94.5) (end 157.5 84.25) (width 0.2) (layer "F.Cu") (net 4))
 (segment (start 157.5 80.75) (end 156.65 79.9) (width 0.2) (layer "F.Cu") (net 4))
 (segment (start 146.25 93.4625) (end 146.25 94.25) (width 0.2) (layer "F.Cu") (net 4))
 (segment (start 144.8 93.9125) (end 145.25 93.4625) (width 0.2) (layer "F.Cu") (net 6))
 (segment (start 144.8 95.05) (end 144.8 93.9125) (width 0.2) (layer "F.Cu") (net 6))
 (via (at 144.8 95.05) (size 0.7) (drill 0.3) (layers "F.Cu" "B.Cu") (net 6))
 (segment (start 159 82.5) (end 157.855 81.355) (width 0.2) (layer "B.Cu") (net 6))
 (segment (start 159 86) (end 159 82.5) (width 0.2) (layer "B.Cu") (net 6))
 (segment (start 157.855 81.355) (end 156.265 81.355) (width 0.2) (layer "B.Cu") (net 6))
 (segment (start 144.8 95.05) (end 145.25 95.5) (width 0.2) (layer "B.Cu") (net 6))
 (segment (start 149.5 95.5) (end 159 86) (width 0.2) (layer "B.Cu") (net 6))
 (segment (start 145.25 95.5) (end 149.5 95.5) (width 0.2) (layer "B.Cu") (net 6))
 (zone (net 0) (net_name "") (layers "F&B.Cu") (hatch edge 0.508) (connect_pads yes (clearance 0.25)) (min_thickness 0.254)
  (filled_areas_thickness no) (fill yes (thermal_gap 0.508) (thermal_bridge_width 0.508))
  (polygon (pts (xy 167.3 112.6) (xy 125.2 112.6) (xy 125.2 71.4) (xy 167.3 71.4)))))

